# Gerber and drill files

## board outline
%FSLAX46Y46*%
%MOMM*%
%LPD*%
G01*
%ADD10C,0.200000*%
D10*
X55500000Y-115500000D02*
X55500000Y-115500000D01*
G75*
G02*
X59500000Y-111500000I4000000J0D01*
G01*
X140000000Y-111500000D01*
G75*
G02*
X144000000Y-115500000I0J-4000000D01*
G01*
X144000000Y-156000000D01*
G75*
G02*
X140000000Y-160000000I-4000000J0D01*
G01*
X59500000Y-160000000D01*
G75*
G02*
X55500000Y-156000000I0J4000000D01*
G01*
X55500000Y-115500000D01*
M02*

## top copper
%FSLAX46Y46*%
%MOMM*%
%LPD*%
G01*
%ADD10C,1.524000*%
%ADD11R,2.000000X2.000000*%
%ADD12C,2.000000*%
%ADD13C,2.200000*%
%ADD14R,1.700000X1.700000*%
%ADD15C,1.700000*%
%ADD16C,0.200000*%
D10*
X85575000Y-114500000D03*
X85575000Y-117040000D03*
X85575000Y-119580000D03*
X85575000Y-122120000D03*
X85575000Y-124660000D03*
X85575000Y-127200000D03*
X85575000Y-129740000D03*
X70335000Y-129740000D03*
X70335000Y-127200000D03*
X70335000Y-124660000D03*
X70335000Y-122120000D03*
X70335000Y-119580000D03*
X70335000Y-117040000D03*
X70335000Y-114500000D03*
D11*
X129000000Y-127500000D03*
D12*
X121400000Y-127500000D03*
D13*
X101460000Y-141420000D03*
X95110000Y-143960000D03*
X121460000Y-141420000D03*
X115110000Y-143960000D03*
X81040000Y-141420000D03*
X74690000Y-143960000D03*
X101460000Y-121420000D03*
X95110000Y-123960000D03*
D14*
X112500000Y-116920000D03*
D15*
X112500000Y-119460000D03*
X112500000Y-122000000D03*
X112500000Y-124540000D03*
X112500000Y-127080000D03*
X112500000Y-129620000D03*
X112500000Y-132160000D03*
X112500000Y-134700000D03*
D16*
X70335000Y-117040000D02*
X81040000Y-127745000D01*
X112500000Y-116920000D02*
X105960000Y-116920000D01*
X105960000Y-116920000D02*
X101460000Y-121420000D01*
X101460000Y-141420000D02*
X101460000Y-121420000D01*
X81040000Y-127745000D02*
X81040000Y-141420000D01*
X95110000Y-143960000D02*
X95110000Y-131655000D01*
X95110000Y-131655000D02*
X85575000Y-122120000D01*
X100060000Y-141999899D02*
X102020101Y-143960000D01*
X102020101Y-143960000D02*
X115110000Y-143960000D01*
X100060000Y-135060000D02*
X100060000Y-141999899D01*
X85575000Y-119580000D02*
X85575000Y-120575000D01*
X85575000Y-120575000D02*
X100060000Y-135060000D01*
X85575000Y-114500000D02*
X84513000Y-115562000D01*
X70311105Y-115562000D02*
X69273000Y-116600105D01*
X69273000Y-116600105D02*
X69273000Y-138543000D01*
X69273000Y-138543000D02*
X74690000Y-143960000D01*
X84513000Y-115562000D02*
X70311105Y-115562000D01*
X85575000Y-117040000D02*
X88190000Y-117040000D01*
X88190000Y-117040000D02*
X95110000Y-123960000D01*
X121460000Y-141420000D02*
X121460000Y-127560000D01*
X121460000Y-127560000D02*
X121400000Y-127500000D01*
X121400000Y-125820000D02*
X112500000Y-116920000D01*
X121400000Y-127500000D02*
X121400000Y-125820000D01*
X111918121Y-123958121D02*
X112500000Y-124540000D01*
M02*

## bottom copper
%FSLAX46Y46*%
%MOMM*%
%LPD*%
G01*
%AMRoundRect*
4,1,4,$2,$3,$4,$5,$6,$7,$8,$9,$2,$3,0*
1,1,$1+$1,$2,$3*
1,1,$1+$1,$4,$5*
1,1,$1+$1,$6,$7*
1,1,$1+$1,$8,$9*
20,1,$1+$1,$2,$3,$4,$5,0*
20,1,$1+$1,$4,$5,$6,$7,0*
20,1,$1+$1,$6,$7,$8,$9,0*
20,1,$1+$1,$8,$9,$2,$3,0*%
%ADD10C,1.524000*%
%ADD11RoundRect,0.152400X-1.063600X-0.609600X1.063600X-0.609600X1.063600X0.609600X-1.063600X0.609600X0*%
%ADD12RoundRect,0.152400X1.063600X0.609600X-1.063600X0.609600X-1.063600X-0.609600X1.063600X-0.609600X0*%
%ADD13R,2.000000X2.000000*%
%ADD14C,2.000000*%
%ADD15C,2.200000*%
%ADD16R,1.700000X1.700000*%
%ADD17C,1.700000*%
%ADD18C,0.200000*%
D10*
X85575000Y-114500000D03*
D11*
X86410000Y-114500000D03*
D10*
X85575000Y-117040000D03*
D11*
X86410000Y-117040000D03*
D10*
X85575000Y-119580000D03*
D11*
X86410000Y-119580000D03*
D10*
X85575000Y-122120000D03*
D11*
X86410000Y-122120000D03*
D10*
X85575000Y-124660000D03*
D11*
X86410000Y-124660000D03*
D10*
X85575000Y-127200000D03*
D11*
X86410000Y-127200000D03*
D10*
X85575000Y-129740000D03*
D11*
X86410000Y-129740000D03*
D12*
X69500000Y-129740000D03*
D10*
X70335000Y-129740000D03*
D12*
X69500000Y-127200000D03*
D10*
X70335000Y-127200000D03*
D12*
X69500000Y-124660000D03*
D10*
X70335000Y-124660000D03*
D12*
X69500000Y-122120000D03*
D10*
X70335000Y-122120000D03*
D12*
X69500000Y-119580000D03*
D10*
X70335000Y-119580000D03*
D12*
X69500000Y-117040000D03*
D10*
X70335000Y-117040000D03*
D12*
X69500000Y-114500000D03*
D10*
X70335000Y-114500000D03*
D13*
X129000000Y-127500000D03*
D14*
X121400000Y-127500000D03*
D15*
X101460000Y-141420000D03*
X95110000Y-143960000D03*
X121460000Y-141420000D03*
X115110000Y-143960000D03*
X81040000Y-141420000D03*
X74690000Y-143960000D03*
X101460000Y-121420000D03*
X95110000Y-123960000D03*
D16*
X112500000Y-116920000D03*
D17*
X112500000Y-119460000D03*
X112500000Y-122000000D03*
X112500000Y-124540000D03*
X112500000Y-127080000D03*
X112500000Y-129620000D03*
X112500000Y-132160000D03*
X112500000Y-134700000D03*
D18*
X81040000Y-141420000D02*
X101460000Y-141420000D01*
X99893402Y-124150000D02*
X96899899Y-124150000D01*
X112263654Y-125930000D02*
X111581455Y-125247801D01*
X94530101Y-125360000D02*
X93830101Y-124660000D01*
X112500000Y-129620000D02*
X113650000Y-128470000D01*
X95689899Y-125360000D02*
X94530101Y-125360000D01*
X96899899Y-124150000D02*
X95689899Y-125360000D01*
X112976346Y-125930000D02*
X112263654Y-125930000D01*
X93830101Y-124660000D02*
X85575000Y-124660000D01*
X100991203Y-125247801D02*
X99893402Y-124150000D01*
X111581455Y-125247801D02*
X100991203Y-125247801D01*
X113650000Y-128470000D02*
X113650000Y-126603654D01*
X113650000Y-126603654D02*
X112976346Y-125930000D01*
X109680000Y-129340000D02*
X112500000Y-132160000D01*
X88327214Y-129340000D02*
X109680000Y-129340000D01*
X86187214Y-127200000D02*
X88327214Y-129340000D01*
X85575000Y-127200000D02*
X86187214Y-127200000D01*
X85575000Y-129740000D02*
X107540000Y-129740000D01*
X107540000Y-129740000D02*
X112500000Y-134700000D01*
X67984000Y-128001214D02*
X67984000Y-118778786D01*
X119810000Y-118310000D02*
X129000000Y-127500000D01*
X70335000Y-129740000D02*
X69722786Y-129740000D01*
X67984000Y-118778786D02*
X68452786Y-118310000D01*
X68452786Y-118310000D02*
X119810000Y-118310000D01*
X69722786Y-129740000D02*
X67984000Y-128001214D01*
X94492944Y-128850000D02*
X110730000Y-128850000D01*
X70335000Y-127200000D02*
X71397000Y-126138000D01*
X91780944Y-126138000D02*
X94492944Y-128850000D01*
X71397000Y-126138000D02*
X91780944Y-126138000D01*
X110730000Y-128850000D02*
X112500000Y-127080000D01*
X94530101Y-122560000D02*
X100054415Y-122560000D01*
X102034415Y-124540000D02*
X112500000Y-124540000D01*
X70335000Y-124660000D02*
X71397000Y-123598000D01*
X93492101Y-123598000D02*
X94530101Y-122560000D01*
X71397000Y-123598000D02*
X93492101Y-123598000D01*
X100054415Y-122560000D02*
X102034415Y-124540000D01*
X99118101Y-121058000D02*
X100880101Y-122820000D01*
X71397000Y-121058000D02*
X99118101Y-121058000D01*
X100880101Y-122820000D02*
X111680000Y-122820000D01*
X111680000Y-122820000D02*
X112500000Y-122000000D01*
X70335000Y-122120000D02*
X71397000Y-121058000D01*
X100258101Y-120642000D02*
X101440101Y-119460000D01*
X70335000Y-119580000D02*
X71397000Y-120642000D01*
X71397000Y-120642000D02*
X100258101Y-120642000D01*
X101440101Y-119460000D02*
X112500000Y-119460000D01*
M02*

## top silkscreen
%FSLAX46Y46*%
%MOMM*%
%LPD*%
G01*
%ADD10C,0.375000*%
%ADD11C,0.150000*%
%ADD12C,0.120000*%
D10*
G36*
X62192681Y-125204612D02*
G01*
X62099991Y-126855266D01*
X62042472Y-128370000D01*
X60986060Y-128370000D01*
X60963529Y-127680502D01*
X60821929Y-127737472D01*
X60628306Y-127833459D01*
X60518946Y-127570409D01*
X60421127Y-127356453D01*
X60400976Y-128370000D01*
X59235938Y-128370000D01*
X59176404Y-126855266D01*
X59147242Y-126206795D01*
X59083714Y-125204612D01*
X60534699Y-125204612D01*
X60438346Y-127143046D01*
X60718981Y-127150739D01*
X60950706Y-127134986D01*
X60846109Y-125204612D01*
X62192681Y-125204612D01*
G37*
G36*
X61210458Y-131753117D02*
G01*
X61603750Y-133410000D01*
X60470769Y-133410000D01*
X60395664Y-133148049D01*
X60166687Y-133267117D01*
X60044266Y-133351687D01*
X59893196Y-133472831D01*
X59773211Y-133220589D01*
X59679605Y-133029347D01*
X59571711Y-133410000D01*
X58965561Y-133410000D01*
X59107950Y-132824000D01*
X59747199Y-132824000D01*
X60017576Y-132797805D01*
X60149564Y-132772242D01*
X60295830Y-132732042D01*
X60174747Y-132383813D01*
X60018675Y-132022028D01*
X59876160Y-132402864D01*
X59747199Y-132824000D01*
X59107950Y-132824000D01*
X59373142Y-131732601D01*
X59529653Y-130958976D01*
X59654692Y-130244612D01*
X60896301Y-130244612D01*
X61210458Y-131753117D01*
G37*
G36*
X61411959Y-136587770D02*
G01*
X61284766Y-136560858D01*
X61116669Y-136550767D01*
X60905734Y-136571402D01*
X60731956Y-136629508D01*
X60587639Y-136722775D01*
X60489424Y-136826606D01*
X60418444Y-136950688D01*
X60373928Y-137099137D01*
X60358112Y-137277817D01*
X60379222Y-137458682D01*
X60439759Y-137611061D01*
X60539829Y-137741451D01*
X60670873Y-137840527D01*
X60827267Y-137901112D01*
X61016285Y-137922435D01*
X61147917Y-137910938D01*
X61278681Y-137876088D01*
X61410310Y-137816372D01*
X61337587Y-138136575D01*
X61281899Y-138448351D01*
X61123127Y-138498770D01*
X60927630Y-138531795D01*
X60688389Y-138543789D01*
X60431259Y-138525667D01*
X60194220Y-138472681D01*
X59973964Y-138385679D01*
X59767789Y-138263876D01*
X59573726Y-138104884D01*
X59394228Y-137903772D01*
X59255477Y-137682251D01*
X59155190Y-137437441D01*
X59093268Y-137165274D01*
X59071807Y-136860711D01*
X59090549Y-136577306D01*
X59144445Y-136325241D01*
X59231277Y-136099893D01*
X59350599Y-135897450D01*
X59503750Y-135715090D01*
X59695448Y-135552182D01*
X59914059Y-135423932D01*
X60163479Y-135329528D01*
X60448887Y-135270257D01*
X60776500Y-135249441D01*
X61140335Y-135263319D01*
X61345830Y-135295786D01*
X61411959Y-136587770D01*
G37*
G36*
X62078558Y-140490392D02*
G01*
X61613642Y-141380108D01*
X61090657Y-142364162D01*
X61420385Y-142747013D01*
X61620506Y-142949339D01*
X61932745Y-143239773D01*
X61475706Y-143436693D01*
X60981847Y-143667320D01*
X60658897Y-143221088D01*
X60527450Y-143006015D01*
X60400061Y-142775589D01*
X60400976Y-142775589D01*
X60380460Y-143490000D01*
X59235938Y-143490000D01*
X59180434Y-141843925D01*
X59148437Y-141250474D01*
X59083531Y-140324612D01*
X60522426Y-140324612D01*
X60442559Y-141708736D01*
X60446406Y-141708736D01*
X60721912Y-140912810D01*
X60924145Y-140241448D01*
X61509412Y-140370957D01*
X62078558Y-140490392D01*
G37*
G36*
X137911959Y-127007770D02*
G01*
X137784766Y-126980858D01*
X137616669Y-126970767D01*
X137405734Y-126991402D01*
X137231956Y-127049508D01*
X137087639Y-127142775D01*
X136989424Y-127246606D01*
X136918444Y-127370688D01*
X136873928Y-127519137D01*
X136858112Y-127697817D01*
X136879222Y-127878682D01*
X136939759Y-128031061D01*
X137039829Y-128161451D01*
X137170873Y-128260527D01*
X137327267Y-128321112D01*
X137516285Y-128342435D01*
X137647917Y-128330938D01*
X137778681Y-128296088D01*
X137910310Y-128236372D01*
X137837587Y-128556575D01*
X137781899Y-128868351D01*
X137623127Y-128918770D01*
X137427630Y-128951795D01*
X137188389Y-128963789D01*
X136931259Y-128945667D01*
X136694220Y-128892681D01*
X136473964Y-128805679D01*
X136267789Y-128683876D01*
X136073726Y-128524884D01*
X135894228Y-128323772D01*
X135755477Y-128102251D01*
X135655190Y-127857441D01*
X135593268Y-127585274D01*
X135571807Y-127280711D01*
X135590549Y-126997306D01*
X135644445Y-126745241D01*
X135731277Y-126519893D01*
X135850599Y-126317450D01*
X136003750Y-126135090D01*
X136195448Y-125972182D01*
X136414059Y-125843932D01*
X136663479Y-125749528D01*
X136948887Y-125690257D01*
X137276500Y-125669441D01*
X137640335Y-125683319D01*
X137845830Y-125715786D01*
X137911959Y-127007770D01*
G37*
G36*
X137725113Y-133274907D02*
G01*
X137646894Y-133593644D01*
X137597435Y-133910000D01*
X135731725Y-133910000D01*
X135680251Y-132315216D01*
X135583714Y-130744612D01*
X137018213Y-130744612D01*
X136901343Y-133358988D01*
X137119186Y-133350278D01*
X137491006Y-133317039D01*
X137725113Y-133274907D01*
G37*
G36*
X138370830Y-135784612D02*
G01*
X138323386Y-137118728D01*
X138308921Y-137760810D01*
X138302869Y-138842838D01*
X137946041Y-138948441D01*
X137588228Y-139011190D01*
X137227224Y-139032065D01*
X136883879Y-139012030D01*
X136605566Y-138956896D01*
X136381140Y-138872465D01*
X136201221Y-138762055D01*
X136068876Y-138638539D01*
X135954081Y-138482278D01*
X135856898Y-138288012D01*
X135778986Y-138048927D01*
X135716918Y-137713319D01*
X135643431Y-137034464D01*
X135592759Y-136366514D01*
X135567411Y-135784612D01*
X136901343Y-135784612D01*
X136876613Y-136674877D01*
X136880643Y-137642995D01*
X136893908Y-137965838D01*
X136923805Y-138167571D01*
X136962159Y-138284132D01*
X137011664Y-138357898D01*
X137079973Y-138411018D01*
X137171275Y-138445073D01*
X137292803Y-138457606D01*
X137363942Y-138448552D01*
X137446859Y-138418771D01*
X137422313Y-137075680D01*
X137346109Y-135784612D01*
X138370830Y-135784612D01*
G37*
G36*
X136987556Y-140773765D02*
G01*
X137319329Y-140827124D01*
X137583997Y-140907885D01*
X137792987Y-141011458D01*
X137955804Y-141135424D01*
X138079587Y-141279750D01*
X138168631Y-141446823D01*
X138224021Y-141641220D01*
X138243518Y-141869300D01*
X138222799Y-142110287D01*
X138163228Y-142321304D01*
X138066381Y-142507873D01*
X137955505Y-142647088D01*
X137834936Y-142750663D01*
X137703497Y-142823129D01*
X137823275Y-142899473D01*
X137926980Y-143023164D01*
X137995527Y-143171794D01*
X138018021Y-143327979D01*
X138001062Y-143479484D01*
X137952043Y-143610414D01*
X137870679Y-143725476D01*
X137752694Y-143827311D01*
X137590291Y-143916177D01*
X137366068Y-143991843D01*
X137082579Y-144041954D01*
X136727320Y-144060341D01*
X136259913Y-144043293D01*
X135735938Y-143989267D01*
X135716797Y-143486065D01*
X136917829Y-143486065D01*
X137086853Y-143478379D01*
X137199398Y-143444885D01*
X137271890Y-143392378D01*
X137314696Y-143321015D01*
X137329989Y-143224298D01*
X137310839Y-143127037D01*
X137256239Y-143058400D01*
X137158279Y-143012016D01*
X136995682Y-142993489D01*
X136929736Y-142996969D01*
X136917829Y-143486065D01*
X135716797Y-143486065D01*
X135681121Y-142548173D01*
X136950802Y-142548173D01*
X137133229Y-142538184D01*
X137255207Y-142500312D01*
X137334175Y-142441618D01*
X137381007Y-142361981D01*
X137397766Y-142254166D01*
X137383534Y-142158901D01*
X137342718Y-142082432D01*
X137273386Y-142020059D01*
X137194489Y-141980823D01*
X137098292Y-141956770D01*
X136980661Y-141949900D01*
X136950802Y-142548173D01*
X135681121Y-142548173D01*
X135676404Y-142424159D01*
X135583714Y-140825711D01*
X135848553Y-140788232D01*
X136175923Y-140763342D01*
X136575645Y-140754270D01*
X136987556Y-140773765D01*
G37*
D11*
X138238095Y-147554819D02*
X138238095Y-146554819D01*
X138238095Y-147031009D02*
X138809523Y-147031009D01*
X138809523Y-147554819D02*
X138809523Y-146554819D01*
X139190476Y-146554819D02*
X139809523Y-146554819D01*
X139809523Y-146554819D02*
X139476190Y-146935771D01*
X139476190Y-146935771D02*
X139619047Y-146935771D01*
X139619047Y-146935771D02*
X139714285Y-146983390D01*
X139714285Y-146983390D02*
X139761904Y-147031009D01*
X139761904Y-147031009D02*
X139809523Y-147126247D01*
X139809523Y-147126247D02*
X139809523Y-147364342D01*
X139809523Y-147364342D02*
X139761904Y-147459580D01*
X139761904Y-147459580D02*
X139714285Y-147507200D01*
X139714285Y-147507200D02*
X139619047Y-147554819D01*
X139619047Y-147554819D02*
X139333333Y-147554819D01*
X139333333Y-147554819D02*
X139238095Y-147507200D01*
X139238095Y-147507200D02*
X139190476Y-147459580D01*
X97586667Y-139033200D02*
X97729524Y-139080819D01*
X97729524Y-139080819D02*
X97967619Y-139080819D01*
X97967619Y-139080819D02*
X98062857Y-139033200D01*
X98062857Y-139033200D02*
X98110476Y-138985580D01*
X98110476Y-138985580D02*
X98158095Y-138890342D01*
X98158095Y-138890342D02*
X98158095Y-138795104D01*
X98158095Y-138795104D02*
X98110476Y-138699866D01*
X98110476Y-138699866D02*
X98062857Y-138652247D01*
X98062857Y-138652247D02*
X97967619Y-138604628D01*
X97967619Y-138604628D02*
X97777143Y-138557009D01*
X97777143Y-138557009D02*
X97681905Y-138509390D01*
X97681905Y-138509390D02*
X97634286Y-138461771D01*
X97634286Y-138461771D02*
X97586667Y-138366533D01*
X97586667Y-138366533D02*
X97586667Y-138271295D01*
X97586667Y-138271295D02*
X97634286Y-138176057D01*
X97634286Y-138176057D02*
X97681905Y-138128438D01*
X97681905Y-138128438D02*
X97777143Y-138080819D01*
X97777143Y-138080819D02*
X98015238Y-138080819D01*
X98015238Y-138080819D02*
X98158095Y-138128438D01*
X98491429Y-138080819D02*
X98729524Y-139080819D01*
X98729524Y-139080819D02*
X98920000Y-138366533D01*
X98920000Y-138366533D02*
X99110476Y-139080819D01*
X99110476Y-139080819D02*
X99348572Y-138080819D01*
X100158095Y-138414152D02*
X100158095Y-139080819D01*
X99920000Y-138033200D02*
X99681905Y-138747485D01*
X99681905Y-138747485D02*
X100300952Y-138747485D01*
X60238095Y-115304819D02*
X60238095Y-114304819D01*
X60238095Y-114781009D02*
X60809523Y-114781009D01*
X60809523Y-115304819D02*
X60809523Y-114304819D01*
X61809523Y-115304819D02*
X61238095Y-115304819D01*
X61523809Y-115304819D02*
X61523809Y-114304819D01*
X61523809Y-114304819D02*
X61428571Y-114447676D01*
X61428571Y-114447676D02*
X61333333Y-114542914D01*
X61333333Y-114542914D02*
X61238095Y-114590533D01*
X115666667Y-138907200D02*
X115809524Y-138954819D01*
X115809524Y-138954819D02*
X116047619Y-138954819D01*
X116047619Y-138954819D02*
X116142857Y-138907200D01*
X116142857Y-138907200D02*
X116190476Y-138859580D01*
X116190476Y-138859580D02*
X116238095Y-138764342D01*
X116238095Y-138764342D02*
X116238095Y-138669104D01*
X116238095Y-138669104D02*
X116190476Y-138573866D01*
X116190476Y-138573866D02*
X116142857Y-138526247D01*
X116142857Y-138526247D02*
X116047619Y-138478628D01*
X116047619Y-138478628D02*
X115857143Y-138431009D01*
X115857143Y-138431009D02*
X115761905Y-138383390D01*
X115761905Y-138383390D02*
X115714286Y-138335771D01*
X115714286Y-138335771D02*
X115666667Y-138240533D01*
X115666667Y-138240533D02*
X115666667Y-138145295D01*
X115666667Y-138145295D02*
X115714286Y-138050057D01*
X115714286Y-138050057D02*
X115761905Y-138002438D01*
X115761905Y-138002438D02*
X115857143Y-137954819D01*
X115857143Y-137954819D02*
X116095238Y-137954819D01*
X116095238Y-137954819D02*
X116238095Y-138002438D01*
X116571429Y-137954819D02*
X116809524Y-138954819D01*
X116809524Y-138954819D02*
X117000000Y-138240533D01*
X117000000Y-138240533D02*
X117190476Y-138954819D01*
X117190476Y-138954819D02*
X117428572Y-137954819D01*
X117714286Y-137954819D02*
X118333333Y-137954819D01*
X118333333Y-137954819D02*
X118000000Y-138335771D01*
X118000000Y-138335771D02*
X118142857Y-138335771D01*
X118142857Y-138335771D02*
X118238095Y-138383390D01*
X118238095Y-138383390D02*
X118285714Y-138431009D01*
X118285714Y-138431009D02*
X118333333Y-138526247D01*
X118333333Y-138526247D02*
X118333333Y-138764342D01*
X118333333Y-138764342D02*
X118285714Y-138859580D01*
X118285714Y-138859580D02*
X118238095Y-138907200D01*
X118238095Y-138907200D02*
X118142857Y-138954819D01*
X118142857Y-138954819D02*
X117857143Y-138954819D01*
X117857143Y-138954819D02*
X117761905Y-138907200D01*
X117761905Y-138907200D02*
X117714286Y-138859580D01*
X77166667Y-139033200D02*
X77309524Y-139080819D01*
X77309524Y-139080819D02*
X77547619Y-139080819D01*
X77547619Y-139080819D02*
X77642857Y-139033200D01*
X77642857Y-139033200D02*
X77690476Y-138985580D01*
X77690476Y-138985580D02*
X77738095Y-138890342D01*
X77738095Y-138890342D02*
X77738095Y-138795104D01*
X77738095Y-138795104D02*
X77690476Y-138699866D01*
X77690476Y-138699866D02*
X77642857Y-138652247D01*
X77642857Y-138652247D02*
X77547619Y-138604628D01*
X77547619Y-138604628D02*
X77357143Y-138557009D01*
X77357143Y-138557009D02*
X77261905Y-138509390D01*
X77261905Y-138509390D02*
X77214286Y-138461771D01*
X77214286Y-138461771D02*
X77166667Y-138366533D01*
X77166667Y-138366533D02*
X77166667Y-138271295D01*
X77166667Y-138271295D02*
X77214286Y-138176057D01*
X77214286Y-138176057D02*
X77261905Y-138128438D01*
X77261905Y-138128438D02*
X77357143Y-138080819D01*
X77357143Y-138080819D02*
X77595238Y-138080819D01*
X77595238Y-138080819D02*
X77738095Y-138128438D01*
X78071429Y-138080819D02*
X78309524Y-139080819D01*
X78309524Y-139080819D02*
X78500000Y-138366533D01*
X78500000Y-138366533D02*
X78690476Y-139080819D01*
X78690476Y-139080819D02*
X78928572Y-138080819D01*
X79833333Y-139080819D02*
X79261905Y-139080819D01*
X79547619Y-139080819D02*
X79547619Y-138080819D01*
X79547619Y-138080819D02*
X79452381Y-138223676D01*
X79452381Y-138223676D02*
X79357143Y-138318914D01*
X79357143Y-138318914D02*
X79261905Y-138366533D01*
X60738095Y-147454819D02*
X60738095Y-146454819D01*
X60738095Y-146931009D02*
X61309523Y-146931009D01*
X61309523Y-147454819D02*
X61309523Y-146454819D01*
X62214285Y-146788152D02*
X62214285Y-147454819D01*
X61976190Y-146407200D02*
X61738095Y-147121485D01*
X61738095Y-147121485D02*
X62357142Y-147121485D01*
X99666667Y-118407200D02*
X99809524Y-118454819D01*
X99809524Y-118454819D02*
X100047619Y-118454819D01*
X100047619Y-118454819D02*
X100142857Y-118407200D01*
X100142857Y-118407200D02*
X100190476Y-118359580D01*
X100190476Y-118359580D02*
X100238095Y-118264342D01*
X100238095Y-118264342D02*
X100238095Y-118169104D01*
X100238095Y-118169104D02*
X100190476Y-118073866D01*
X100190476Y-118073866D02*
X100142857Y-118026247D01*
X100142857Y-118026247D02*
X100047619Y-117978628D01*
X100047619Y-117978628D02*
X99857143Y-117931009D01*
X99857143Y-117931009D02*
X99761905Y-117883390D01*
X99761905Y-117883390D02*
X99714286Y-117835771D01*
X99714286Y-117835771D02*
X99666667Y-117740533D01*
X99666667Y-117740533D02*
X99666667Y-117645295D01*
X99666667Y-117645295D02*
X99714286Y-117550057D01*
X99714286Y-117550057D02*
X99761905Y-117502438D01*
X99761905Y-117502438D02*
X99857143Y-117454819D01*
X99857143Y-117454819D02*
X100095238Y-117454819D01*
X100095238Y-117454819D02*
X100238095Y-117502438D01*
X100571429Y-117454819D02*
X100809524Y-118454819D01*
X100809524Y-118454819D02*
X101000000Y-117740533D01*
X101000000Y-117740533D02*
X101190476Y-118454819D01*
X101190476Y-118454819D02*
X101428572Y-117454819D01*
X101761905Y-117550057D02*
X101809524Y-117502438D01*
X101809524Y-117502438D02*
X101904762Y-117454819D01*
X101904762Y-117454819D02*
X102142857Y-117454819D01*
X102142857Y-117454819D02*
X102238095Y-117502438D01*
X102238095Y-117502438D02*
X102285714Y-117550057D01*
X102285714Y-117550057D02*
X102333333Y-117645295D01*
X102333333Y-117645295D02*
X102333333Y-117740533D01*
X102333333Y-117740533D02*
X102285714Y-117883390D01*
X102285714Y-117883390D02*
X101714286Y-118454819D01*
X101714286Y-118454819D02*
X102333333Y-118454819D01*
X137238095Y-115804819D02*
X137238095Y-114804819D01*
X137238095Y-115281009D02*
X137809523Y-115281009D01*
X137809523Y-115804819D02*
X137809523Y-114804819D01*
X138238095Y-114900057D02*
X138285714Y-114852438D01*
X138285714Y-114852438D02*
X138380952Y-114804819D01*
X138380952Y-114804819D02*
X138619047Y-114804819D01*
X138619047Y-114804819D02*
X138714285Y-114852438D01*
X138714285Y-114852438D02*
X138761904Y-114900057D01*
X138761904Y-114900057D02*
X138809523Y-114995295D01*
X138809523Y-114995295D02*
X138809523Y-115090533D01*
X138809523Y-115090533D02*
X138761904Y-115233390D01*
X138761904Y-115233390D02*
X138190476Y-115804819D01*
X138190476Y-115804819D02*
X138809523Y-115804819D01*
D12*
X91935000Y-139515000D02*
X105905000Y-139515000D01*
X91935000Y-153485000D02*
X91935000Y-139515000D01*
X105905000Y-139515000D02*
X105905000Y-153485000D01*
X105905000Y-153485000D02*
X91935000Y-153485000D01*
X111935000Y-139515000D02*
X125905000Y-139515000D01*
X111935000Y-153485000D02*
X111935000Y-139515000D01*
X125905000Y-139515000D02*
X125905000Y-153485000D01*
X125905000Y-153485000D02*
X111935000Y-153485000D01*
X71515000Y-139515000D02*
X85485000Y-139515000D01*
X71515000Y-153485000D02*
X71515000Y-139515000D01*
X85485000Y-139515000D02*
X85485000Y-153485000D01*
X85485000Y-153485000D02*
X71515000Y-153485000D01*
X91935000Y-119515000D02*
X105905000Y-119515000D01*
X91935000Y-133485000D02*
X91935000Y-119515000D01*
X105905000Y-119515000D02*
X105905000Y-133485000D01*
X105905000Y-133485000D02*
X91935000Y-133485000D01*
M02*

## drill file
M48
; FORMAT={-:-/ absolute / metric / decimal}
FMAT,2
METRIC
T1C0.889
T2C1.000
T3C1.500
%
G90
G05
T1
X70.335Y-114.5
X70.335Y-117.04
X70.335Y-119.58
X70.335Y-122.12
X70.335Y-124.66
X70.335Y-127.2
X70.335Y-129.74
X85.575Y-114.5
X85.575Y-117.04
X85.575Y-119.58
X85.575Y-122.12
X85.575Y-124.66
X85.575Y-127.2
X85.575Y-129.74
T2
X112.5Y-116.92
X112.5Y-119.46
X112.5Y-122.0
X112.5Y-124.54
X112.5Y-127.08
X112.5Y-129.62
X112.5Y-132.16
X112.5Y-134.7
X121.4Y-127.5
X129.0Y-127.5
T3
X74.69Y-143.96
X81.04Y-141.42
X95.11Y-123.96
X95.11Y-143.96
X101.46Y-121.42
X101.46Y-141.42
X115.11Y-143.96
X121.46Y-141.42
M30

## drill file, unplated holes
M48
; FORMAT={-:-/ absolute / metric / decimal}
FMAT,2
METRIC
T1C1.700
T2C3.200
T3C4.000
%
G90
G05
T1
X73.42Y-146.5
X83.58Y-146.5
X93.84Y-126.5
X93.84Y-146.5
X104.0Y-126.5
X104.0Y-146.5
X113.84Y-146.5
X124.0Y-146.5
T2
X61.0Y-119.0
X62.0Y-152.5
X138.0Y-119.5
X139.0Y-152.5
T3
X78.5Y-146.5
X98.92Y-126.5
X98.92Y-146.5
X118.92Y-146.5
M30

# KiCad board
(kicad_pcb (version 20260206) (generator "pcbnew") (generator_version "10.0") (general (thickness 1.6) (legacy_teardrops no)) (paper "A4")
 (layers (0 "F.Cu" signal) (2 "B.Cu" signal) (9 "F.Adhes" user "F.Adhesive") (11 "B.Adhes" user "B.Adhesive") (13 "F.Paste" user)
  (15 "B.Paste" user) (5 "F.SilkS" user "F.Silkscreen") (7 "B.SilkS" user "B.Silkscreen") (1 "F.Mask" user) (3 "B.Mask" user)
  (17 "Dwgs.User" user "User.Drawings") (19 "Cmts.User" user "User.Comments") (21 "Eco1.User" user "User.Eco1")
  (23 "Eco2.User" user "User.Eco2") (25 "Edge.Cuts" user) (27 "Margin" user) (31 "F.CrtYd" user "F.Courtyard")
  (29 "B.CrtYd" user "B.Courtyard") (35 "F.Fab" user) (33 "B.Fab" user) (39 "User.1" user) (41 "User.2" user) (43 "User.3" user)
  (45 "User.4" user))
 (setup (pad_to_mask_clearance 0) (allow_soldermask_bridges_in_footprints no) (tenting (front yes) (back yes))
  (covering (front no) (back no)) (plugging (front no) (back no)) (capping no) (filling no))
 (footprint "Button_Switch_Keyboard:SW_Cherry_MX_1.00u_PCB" (layer "F.Cu") (at 101.46 141.42)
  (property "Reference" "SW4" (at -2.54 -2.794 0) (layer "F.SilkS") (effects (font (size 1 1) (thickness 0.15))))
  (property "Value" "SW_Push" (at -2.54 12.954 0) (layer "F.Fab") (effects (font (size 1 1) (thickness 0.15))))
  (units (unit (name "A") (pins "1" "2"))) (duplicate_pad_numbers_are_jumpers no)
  (fp_line (start -9.525 -1.905) (end 4.445 -1.905) (stroke (width 0.12) (type solid)) (layer "F.SilkS"))
  (fp_line (start -9.525 12.065) (end -9.525 -1.905) (stroke (width 0.12) (type solid)) (layer "F.SilkS"))
  (fp_line (start 4.445 -1.905) (end 4.445 12.065) (stroke (width 0.12) (type solid)) (layer "F.SilkS"))
  (fp_line (start 4.445 12.065) (end -9.525 12.065) (stroke (width 0.12) (type solid)) (layer "F.SilkS"))
  (pad "" np_thru_hole circle (at -7.62 5.08) (size 1.7 1.7) (drill 1.7) (layers "*.Cu" "*.Mask"))
  (pad "" np_thru_hole circle (at -2.54 5.08) (size 4 4) (drill 4) (layers "*.Cu" "*.Mask"))
  (pad "" np_thru_hole circle (at 2.54 5.08) (size 1.7 1.7) (drill 1.7) (layers "*.Cu" "*.Mask"))
  (pad "1" thru_hole circle (at 0 0) (size 2.2 2.2) (drill 1.5) (layers "*.Cu" "*.Mask") (remove_unused_layers no) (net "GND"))
  (pad "2" thru_hole circle (at -6.35 2.54) (size 2.2 2.2) (drill 1.5) (layers "*.Cu" "*.Mask") (remove_unused_layers no)
   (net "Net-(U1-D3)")))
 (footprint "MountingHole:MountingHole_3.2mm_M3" (layer "F.Cu") (at 139 152.5)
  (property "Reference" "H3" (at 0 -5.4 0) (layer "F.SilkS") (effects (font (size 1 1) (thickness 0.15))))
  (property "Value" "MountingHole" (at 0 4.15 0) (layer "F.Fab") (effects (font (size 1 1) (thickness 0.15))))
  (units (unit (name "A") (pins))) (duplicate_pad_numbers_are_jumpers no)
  (pad "" np_thru_hole circle (at 0 0) (size 3.2 3.2) (drill 3.2) (layers "*.Cu" "*.Mask")))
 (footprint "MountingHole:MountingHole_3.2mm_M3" (layer "F.Cu") (at 61 119)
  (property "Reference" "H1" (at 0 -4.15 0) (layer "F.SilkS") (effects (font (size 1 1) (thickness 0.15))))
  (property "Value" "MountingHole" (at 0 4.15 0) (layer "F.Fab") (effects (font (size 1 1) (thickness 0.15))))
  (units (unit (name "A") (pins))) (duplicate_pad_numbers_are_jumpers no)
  (pad "" np_thru_hole circle (at 0 0) (size 3.2 3.2) (drill 3.2) (layers "*.Cu" "*.Mask")))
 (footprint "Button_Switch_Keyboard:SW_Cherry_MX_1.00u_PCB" (layer "F.Cu") (at 121.46 141.42)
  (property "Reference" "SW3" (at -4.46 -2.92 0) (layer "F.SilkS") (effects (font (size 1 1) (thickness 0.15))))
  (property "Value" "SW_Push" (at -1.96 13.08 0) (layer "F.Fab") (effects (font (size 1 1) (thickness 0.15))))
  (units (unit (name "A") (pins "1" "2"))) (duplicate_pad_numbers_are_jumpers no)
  (fp_line (start -9.525 -1.905) (end 4.445 -1.905) (stroke (width 0.12) (type solid)) (layer "F.SilkS"))
  (fp_line (start -9.525 12.065) (end -9.525 -1.905) (stroke (width 0.12) (type solid)) (layer "F.SilkS"))
  (fp_line (start 4.445 -1.905) (end 4.445 12.065) (stroke (width 0.12) (type solid)) (layer "F.SilkS"))
  (fp_line (start 4.445 12.065) (end -9.525 12.065) (stroke (width 0.12) (type solid)) (layer "F.SilkS"))
  (pad "" np_thru_hole circle (at -7.62 5.08) (size 1.7 1.7) (drill 1.7) (layers "*.Cu" "*.Mask"))
  (pad "" np_thru_hole circle (at -2.54 5.08) (size 4 4) (drill 4) (layers "*.Cu" "*.Mask"))
  (pad "" np_thru_hole circle (at 2.54 5.08) (size 1.7 1.7) (drill 1.7) (layers "*.Cu" "*.Mask"))
  (pad "1" thru_hole circle (at 0 0) (size 2.2 2.2) (drill 1.5) (layers "*.Cu" "*.Mask") (remove_unused_layers no) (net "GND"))
  (pad "2" thru_hole circle (at -6.35 2.54) (size 2.2 2.2) (drill 1.5) (layers "*.Cu" "*.Mask") (remove_unused_layers no)
   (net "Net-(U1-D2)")))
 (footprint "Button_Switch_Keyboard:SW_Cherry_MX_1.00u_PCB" (layer "F.Cu") (at 81.04 141.42)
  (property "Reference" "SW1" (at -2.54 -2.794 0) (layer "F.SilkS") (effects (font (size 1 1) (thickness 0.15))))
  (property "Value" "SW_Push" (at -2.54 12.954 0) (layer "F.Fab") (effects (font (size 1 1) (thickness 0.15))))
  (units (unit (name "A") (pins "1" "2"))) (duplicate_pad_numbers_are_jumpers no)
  (fp_line (start -9.525 -1.905) (end 4.445 -1.905) (stroke (width 0.12) (type solid)) (layer "F.SilkS"))
  (fp_line (start -9.525 12.065) (end -9.525 -1.905) (stroke (width 0.12) (type solid)) (layer "F.SilkS"))
  (fp_line (start 4.445 -1.905) (end 4.445 12.065) (stroke (width 0.12) (type solid)) (layer "F.SilkS"))
  (fp_line (start 4.445 12.065) (end -9.525 12.065) (stroke (width 0.12) (type solid)) (layer "F.SilkS"))
  (pad "" np_thru_hole circle (at -7.62 5.08) (size 1.7 1.7) (drill 1.7) (layers "*.Cu" "*.Mask"))
  (pad "" np_thru_hole circle (at -2.54 5.08) (size 4 4) (drill 4) (layers "*.Cu" "*.Mask"))
  (pad "" np_thru_hole circle (at 2.54 5.08) (size 1.7 1.7) (drill 1.7) (layers "*.Cu" "*.Mask"))
  (pad "1" thru_hole circle (at 0 0) (size 2.2 2.2) (drill 1.5) (layers "*.Cu" "*.Mask") (remove_unused_layers no) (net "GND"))
  (pad "2" thru_hole circle (at -6.35 2.54) (size 2.2 2.2) (drill 1.5) (layers "*.Cu" "*.Mask") (remove_unused_layers no)
   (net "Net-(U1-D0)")))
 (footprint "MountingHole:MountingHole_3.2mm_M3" (layer "F.Cu") (at 62 152.5)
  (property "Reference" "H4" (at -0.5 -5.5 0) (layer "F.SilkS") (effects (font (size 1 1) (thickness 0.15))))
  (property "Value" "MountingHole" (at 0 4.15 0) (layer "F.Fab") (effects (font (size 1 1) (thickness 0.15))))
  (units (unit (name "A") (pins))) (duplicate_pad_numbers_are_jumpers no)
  (pad "" np_thru_hole circle (at 0 0) (size 3.2 3.2) (drill 3.2) (layers "*.Cu" "*.Mask")))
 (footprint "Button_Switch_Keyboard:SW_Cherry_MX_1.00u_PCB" (layer "F.Cu") (at 101.46 121.42)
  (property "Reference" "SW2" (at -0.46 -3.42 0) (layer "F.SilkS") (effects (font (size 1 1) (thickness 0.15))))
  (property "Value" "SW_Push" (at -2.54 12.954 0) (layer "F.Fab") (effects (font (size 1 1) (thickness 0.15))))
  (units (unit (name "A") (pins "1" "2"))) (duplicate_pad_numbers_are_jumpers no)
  (fp_line (start -9.525 -1.905) (end 4.445 -1.905) (stroke (width 0.12) (type solid)) (layer "F.SilkS"))
  (fp_line (start -9.525 12.065) (end -9.525 -1.905) (stroke (width 0.12) (type solid)) (layer "F.SilkS"))
  (fp_line (start 4.445 -1.905) (end 4.445 12.065) (stroke (width 0.12) (type solid)) (layer "F.SilkS"))
  (fp_line (start 4.445 12.065) (end -9.525 12.065) (stroke (width 0.12) (type solid)) (layer "F.SilkS"))
  (pad "" np_thru_hole circle (at -7.62 5.08) (size 1.7 1.7) (drill 1.7) (layers "*.Cu" "*.Mask"))
  (pad "" np_thru_hole circle (at -2.54 5.08) (size 4 4) (drill 4) (layers "*.Cu" "*.Mask"))
  (pad "" np_thru_hole circle (at 2.54 5.08) (size 1.7 1.7) (drill 1.7) (layers "*.Cu" "*.Mask"))
  (pad "1" thru_hole circle (at 0 0) (size 2.2 2.2) (drill 1.5) (layers "*.Cu" "*.Mask") (remove_unused_layers no) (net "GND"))
  (pad "2" thru_hole circle (at -6.35 2.54) (size 2.2 2.2) (drill 1.5) (layers "*.Cu" "*.Mask") (remove_unused_layers no)
   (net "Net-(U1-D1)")))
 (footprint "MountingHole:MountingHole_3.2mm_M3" (layer "F.Cu") (at 138 119.5)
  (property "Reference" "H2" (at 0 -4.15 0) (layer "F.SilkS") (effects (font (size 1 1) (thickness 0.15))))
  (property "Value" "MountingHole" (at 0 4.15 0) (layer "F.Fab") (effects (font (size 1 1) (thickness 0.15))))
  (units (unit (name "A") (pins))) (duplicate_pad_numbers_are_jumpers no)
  (pad "" np_thru_hole circle (at 0 0) (size 3.2 3.2) (drill 3.2) (layers "*.Cu" "*.Mask")))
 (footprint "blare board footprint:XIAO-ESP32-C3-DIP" (layer "B.Cu") (at 77.955 122.12 90)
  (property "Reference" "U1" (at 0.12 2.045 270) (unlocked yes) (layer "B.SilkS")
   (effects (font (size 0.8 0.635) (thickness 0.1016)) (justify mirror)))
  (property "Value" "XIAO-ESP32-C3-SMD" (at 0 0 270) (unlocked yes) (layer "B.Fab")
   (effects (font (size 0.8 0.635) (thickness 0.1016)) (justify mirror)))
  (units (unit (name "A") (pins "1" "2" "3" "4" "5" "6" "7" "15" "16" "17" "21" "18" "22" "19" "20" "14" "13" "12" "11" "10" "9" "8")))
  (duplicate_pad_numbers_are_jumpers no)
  (pad "1" thru_hole circle (at 7.62 7.62) (size 1.524 1.524) (drill 0.889) (layers "*.Cu" "*.Mask") (remove_unused_layers no)
   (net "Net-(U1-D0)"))
  (pad "1" smd roundrect (at 7.62 8.455) (size 2.432 1.524) (layers "B.Cu" "B.Mask") (roundrect_rratio 0.1) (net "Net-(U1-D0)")
   (thermal_bridge_angle 45))
  (pad "2" thru_hole circle (at 5.08 7.62) (size 1.524 1.524) (drill 0.889) (layers "*.Cu" "*.Mask") (remove_unused_layers no)
   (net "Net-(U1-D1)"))
  (pad "2" smd roundrect (at 5.08 8.455) (size 2.432 1.524) (layers "B.Cu" "B.Mask") (roundrect_rratio 0.1) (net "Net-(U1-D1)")
   (thermal_bridge_angle 45))
  (pad "3" thru_hole circle (at 2.54 7.62) (size 1.524 1.524) (drill 0.889) (layers "*.Cu" "*.Mask") (remove_unused_layers no)
   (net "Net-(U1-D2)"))
  (pad "3" smd roundrect (at 2.54 8.455) (size 2.432 1.524) (layers "B.Cu" "B.Mask") (roundrect_rratio 0.1) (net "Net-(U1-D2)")
   (thermal_bridge_angle 45))
  (pad "4" thru_hole circle (at 0 7.62) (size 1.524 1.524) (drill 0.889) (layers "*.Cu" "*.Mask") (remove_unused_layers no)
   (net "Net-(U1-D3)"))
  (pad "4" smd roundrect (at 0 8.455) (size 2.432 1.524) (layers "B.Cu" "B.Mask") (roundrect_rratio 0.1) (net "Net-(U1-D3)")
   (thermal_bridge_angle 45))
  (pad "5" thru_hole circle (at -2.54 7.62) (size 1.524 1.524) (drill 0.889) (layers "*.Cu" "*.Mask") (remove_unused_layers no) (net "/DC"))
  (pad "5" smd roundrect (at -2.54 8.455) (size 2.432 1.524) (layers "B.Cu" "B.Mask") (roundrect_rratio 0.1) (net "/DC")
   (thermal_bridge_angle 45))
  (pad "6" thru_hole circle (at -5.08 7.62) (size 1.524 1.524) (drill 0.889) (layers "*.Cu" "*.Mask") (remove_unused_layers no) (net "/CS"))
  (pad "6" smd roundrect (at -5.08 8.455) (size 2.432 1.524) (layers "B.Cu" "B.Mask") (roundrect_rratio 0.1) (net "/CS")
   (thermal_bridge_angle 45))
  (pad "7" thru_hole circle (at -7.62 7.62) (size 1.524 1.524) (drill 0.889) (layers "*.Cu" "*.Mask") (remove_unused_layers no) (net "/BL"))
  (pad "7" smd roundrect (at -7.62 8.455) (size 2.432 1.524) (layers "B.Cu" "B.Mask") (roundrect_rratio 0.1) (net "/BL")
   (thermal_bridge_angle 45))
  (pad "8" smd roundrect (at -7.62 -8.455 180) (size 2.432 1.524) (layers "B.Cu" "B.Mask") (roundrect_rratio 0.1) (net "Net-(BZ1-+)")
   (thermal_bridge_angle 45))
  (pad "8" thru_hole circle (at -7.62 -7.62 180) (size 1.524 1.524) (drill 0.889) (layers "*.Cu" "*.Mask") (remove_unused_layers no)
   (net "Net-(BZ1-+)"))
  (pad "9" smd roundrect (at -5.08 -8.455 180) (size 2.432 1.524) (layers "B.Cu" "B.Mask") (roundrect_rratio 0.1) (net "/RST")
   (thermal_bridge_angle 45))
  (pad "9" thru_hole circle (at -5.08 -7.62 180) (size 1.524 1.524) (drill 0.889) (layers "*.Cu" "*.Mask") (remove_unused_layers no)
   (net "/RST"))
  (pad "10" smd roundrect (at -2.54 -8.455 180) (size 2.432 1.524) (layers "B.Cu" "B.Mask") (roundrect_rratio 0.1) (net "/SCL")
   (thermal_bridge_angle 45))
  (pad "10" thru_hole circle (at -2.54 -7.62 180) (size 1.524 1.524) (drill 0.889) (layers "*.Cu" "*.Mask") (remove_unused_layers no)
   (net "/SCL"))
  (pad "11" smd roundrect (at 0 -8.455 180) (size 2.432 1.524) (layers "B.Cu" "B.Mask") (roundrect_rratio 0.1) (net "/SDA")
   (thermal_bridge_angle 45))
  (pad "11" thru_hole circle (at 0 -7.62 180) (size 1.524 1.524) (drill 0.889) (layers "*.Cu" "*.Mask") (remove_unused_layers no)
   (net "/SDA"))
  (pad "12" smd roundrect (at 2.54 -8.455 180) (size 2.432 1.524) (layers "B.Cu" "B.Mask") (roundrect_rratio 0.1) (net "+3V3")
   (thermal_bridge_angle 45))
  (pad "12" thru_hole circle (at 2.54 -7.62 180) (size 1.524 1.524) (drill 0.889) (layers "*.Cu" "*.Mask") (remove_unused_layers no)
   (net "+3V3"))
  (pad "13" smd roundrect (at 5.08 -8.455 180) (size 2.432 1.524) (layers "B.Cu" "B.Mask") (roundrect_rratio 0.1) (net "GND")
   (thermal_bridge_angle 45))
  (pad "13" thru_hole circle (at 5.08 -7.62 180) (size 1.524 1.524) (drill 0.889) (layers "*.Cu" "*.Mask") (remove_unused_layers no)
   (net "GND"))
  (pad "14" smd roundrect (at 7.62 -8.455 180) (size 2.432 1.524) (layers "B.Cu" "B.Mask") (roundrect_rratio 0.1)
   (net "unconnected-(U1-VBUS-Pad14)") (thermal_bridge_angle 45))
  (pad "14" thru_hole circle (at 7.62 -7.62 180) (size 1.524 1.524) (drill 0.889) (layers "*.Cu" "*.Mask") (remove_unused_layers no)
   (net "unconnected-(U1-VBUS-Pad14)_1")))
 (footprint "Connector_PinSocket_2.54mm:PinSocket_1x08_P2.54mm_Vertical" (layer "B.Cu") (at 112.5 116.92 180)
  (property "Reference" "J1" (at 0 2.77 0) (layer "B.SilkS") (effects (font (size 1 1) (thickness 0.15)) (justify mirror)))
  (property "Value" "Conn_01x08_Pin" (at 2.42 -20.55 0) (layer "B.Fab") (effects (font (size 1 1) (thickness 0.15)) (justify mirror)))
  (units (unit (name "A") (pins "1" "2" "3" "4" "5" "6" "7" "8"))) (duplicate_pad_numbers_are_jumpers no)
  (pad "1" thru_hole rect (at 0 0 180) (size 1.7 1.7) (drill 1) (layers "*.Cu" "*.Mask") (remove_unused_layers no) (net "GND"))
  (pad "2" thru_hole circle (at 0 -2.54 180) (size 1.7 1.7) (drill 1) (layers "*.Cu" "*.Mask") (remove_unused_layers no) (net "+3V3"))
  (pad "3" thru_hole circle (at 0 -5.08 180) (size 1.7 1.7) (drill 1) (layers "*.Cu" "*.Mask") (remove_unused_layers no) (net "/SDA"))
  (pad "4" thru_hole circle (at 0 -7.62 180) (size 1.7 1.7) (drill 1) (layers "*.Cu" "*.Mask") (remove_unused_layers no) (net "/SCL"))
  (pad "5" thru_hole circle (at 0 -10.16 180) (size 1.7 1.7) (drill 1) (layers "*.Cu" "*.Mask") (remove_unused_layers no) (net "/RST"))
  (pad "6" thru_hole circle (at 0 -12.7 180) (size 1.7 1.7) (drill 1) (layers "*.Cu" "*.Mask") (remove_unused_layers no) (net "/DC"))
  (pad "7" thru_hole circle (at 0 -15.24 180) (size 1.7 1.7) (drill 1) (layers "*.Cu" "*.Mask") (remove_unused_layers no) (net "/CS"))
  (pad "8" thru_hole circle (at 0 -17.78 180) (size 1.7 1.7) (drill 1) (layers "*.Cu" "*.Mask") (remove_unused_layers no) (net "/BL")))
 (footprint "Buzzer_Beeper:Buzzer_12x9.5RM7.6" (layer "B.Cu") (at 129 127.5 180)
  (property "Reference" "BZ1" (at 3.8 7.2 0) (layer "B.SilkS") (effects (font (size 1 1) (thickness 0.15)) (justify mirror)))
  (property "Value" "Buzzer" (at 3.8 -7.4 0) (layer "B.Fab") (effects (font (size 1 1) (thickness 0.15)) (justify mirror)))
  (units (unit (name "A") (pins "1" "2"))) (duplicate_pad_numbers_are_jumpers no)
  (pad "1" thru_hole rect (at 0 0 180) (size 2 2) (drill 1) (layers "*.Cu" "*.Mask") (remove_unused_layers no) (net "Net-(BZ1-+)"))
  (pad "2" thru_hole circle (at 7.6 0 180) (size 2 2) (drill 1) (layers "*.Cu" "*.Mask") (remove_unused_layers no) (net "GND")))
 (gr_rect (start 55.5 111.5) (end 144 160) (radius 4) (stroke (width 0.2) (type default)) (fill no) (layer "Edge.Cuts"))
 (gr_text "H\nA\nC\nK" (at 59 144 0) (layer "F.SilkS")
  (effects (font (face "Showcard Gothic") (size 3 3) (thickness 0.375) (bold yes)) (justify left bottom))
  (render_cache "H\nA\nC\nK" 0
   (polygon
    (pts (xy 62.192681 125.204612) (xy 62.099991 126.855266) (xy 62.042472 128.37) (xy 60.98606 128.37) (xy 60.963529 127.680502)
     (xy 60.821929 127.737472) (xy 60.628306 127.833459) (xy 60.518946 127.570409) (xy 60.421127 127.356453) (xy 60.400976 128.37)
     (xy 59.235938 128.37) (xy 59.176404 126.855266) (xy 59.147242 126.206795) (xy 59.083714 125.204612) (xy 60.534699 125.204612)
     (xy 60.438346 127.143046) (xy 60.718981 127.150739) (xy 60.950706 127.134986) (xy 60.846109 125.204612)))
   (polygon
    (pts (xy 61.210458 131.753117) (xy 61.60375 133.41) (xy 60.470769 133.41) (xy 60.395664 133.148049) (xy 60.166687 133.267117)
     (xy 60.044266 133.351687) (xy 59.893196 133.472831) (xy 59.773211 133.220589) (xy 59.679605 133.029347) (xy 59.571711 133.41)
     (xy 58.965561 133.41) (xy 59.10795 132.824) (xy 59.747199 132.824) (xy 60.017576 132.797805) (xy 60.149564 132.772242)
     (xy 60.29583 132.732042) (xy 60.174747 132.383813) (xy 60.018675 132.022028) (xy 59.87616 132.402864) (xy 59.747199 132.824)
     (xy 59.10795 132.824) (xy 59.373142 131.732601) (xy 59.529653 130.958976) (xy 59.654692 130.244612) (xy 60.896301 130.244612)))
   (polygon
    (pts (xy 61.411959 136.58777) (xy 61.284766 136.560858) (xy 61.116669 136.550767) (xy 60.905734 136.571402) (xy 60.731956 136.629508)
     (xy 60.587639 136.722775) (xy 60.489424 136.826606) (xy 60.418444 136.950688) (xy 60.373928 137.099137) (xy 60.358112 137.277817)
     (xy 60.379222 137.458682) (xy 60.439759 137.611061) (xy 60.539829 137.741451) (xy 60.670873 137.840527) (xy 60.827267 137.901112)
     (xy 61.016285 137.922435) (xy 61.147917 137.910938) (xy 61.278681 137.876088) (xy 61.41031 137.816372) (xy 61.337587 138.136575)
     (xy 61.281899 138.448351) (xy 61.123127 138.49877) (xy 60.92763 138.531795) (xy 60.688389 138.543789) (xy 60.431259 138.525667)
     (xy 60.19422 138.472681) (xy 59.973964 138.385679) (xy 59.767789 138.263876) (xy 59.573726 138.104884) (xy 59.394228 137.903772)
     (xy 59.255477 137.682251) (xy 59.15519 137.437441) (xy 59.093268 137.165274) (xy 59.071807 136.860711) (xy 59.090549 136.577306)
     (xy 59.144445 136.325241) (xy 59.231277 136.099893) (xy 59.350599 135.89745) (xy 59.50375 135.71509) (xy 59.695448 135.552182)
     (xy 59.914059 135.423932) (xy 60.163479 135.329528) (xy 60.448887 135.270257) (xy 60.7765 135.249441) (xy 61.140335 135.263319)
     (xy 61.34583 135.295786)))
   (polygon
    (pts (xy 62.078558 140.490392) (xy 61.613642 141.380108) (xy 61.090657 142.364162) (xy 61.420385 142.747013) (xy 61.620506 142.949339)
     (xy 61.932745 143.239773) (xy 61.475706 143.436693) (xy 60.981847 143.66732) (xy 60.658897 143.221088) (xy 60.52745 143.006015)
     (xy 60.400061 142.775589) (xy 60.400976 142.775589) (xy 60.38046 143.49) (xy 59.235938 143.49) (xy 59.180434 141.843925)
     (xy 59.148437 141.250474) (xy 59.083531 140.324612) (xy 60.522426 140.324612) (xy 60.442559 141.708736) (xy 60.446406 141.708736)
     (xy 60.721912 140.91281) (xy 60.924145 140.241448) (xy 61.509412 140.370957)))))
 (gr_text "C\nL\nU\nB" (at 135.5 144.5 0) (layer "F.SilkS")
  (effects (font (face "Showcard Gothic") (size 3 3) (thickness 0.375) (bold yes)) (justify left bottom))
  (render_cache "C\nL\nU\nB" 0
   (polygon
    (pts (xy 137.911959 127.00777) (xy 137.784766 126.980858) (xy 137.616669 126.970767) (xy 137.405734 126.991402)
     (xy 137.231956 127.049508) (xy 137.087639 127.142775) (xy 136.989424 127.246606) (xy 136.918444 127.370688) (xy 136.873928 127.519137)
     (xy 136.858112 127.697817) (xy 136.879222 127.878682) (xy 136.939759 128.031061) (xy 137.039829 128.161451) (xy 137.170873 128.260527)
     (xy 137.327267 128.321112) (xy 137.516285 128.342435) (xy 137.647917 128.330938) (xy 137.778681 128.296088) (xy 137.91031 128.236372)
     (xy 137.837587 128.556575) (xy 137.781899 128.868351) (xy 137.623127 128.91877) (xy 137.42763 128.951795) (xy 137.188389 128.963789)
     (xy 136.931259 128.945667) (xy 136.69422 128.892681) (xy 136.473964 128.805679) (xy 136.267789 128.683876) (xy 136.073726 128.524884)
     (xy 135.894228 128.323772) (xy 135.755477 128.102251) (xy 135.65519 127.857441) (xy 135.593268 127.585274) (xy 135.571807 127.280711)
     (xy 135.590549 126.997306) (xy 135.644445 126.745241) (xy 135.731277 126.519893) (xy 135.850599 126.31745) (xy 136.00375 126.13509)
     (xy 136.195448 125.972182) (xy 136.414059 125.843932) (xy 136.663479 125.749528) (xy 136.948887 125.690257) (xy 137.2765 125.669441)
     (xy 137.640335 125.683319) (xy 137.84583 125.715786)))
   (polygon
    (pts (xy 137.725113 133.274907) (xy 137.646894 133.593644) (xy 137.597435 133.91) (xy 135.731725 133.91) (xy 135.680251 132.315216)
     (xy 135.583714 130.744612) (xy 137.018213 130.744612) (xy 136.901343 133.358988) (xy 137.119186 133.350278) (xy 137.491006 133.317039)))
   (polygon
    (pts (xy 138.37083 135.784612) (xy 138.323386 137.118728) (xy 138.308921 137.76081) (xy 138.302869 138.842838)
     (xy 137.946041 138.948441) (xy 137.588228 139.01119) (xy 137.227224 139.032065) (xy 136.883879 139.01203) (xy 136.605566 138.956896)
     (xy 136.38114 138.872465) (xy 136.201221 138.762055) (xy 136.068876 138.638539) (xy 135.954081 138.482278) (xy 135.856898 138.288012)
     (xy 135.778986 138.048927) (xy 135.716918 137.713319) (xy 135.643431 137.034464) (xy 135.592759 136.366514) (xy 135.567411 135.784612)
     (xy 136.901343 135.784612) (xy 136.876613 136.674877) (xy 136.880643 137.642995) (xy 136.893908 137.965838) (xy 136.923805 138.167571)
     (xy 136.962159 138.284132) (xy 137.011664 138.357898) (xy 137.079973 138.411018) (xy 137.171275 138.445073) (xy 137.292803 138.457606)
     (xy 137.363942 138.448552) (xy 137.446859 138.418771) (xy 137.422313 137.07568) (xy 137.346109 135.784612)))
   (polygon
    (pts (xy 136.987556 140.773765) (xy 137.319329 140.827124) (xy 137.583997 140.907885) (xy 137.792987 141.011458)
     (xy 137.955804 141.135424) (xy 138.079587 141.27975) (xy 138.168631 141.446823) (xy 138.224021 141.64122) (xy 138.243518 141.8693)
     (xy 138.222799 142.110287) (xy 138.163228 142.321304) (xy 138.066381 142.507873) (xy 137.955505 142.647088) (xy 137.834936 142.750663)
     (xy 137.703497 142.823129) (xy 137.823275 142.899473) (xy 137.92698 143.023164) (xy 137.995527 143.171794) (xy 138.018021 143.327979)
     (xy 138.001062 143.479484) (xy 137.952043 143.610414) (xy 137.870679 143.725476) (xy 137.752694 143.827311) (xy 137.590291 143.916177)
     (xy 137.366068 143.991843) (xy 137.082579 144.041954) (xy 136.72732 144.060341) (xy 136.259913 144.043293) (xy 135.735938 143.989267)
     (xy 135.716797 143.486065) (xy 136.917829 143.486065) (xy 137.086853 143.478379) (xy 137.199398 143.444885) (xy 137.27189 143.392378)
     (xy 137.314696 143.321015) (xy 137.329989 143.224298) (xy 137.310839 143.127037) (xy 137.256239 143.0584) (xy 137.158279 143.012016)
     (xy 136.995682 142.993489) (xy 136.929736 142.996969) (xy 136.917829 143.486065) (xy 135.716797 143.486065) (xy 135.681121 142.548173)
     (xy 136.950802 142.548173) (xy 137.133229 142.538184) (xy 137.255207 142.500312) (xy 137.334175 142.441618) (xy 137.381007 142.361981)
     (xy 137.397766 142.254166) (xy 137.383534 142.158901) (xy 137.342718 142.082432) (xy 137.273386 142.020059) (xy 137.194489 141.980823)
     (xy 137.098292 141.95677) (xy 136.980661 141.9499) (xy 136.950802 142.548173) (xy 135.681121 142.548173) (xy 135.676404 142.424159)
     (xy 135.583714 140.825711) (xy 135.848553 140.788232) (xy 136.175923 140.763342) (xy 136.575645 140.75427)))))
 (segment (start 121.46 141.42) (end 121.46 127.56) (width 0.2) (layer "F.Cu") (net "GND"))
 (segment (start 70.335 117.04) (end 81.04 127.745) (width 0.2) (layer "F.Cu") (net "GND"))
 (segment (start 121.4 127.5) (end 121.4 125.82) (width 0.2) (layer "F.Cu") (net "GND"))
 (segment (start 112.5 116.92) (end 105.96 116.92) (width 0.2) (layer "F.Cu") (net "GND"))
 (segment (start 121.4 125.82) (end 112.5 116.92) (width 0.2) (layer "F.Cu") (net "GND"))
 (segment (start 105.96 116.92) (end 101.46 121.42) (width 0.2) (layer "F.Cu") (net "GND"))
 (segment (start 101.46 141.42) (end 101.46 121.42) (width 0.2) (layer "F.Cu") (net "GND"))
 (segment (start 121.46 127.56) (end 121.4 127.5) (width 0.2) (layer "F.Cu") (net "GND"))
 (segment (start 81.04 127.745) (end 81.04 141.42) (width 0.2) (layer "F.Cu") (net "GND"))
 (segment (start 81.04 141.42) (end 101.46 141.42) (width 0.2) (layer "B.Cu") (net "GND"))
 (segment (start 95.11 143.96) (end 95.11 131.655) (width 0.2) (layer "F.Cu") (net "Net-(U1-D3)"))
 (segment (start 95.11 131.655) (end 85.575 122.12) (width 0.2) (layer "F.Cu") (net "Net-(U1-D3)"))
 (segment (start 100.06 141.999899) (end 102.020101 143.96) (width 0.2) (layer "F.Cu") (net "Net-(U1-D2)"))
 (segment (start 102.020101 143.96) (end 115.11 143.96) (width 0.2) (layer "F.Cu") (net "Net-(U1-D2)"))
 (segment (start 100.06 135.06) (end 100.06 141.999899) (width 0.2) (layer "F.Cu") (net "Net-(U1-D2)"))
 (segment (start 85.575 119.58) (end 85.575 120.575) (width 0.2) (layer "F.Cu") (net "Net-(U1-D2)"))
 (segment (start 85.575 120.575) (end 100.06 135.06) (width 0.2) (layer "F.Cu") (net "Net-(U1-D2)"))
 (segment (start 85.575 114.5) (end 84.513 115.562) (width 0.2) (layer "F.Cu") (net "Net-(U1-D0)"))
 (segment (start 70.311105 115.562) (end 69.273 116.600105) (width 0.2) (layer "F.Cu") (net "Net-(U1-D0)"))
 (segment (start 69.273 116.600105) (end 69.273 138.543) (width 0.2) (layer "F.Cu") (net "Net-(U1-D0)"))
 (segment (start 69.273 138.543) (end 74.69 143.96) (width 0.2) (layer "F.Cu") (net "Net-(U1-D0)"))
 (segment (start 84.513 115.562) (end 70.311105 115.562) (width 0.2) (layer "F.Cu") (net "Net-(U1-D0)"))
 (segment (start 85.575 117.04) (end 88.19 117.04) (width 0.2) (layer "F.Cu") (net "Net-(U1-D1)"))
 (segment (start 88.19 117.04) (end 95.11 123.96) (width 0.2) (layer "F.Cu") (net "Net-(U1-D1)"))
 (segment (start 99.893402 124.15) (end 96.899899 124.15) (width 0.2) (layer "B.Cu") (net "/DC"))
 (segment (start 112.263654 125.93) (end 111.581455 125.247801) (width 0.2) (layer "B.Cu") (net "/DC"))
 (segment (start 94.530101 125.36) (end 93.830101 124.66) (width 0.2) (layer "B.Cu") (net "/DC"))
 (segment (start 112.5 129.62) (end 113.65 128.47) (width 0.2) (layer "B.Cu") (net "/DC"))
 (segment (start 95.689899 125.36) (end 94.530101 125.36) (width 0.2) (layer "B.Cu") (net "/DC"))
 (segment (start 96.899899 124.15) (end 95.689899 125.36) (width 0.2) (layer "B.Cu") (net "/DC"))
 (segment (start 112.976346 125.93) (end 112.263654 125.93) (width 0.2) (layer "B.Cu") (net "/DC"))
 (segment (start 93.830101 124.66) (end 85.575 124.66) (width 0.2) (layer "B.Cu") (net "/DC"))
 (segment (start 100.991203 125.247801) (end 99.893402 124.15) (width 0.2) (layer "B.Cu") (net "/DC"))
 (segment (start 111.581455 125.247801) (end 100.991203 125.247801) (width 0.2) (layer "B.Cu") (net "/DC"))
 (segment (start 113.65 128.47) (end 113.65 126.603654) (width 0.2) (layer "B.Cu") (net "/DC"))
 (segment (start 113.65 126.603654) (end 112.976346 125.93) (width 0.2) (layer "B.Cu") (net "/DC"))
 (segment (start 109.68 129.34) (end 112.5 132.16) (width 0.2) (layer "B.Cu") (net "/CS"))
 (segment (start 88.327214 129.34) (end 109.68 129.34) (width 0.2) (layer "B.Cu") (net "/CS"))
 (segment (start 86.187214 127.2) (end 88.327214 129.34) (width 0.2) (layer "B.Cu") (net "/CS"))
 (segment (start 85.575 127.2) (end 86.187214 127.2) (width 0.2) (layer "B.Cu") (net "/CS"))
 (segment (start 85.575 129.74) (end 107.54 129.74) (width 0.2) (layer "B.Cu") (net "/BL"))
 (segment (start 107.54 129.74) (end 112.5 134.7) (width 0.2) (layer "B.Cu") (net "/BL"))
 (segment (start 67.984 128.001214) (end 67.984 118.778786) (width 0.2) (layer "B.Cu") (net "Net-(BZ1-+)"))
 (segment (start 119.81 118.31) (end 129 127.5) (width 0.2) (layer "B.Cu") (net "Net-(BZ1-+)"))
 (segment (start 70.335 129.74) (end 69.722786 129.74) (width 0.2) (layer "B.Cu") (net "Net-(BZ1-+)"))
 (segment (start 67.984 118.778786) (end 68.452786 118.31) (width 0.2) (layer "B.Cu") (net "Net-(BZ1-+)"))
 (segment (start 68.452786 118.31) (end 119.81 118.31) (width 0.2) (layer "B.Cu") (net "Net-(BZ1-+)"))
 (segment (start 69.722786 129.74) (end 67.984 128.001214) (width 0.2) (layer "B.Cu") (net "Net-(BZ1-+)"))
 (segment (start 94.492944 128.85) (end 110.73 128.85) (width 0.2) (layer "B.Cu") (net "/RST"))
 (segment (start 70.335 127.2) (end 71.397 126.138) (width 0.2) (layer "B.Cu") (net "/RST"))
 (segment (start 91.780944 126.138) (end 94.492944 128.85) (width 0.2) (layer "B.Cu") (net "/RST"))
 (segment (start 71.397 126.138) (end 91.780944 126.138) (width 0.2) (layer "B.Cu") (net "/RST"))
 (segment (start 110.73 128.85) (end 112.5 127.08) (width 0.2) (layer "B.Cu") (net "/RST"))
 (segment (start 111.918121 123.958121) (end 112.5 124.54) (width 0.2) (layer "F.Cu") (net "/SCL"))
 (segment (start 94.530101 122.56) (end 100.054415 122.56) (width 0.2) (layer "B.Cu") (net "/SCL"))
 (segment (start 102.034415 124.54) (end 112.5 124.54) (width 0.2) (layer "B.Cu") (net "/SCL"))
 (segment (start 70.335 124.66) (end 71.397 123.598) (width 0.2) (layer "B.Cu") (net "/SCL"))
 (segment (start 93.492101 123.598) (end 94.530101 122.56) (width 0.2) (layer "B.Cu") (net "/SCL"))
 (segment (start 71.397 123.598) (end 93.492101 123.598) (width 0.2) (layer "B.Cu") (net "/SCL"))
 (segment (start 100.054415 122.56) (end 102.034415 124.54) (width 0.2) (layer "B.Cu") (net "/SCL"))
 (segment (start 99.118101 121.058) (end 100.880101 122.82) (width 0.2) (layer "B.Cu") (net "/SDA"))
 (segment (start 71.397 121.058) (end 99.118101 121.058) (width 0.2) (layer "B.Cu") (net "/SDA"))
 (segment (start 100.880101 122.82) (end 111.68 122.82) (width 0.2) (layer "B.Cu") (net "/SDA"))
 (segment (start 111.68 122.82) (end 112.5 122) (width 0.2) (layer "B.Cu") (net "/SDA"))
 (segment (start 70.335 122.12) (end 71.397 121.058) (width 0.2) (layer "B.Cu") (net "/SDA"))
 (segment (start 100.258101 120.642) (end 101.440101 119.46) (width 0.2) (layer "B.Cu") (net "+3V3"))
 (segment (start 70.335 119.58) (end 71.397 120.642) (width 0.2) (layer "B.Cu") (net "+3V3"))
 (segment (start 71.397 120.642) (end 100.258101 120.642) (width 0.2) (layer "B.Cu") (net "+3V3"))
 (segment (start 101.440101 119.46) (end 112.5 119.46) (width 0.2) (layer "B.Cu") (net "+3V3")))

